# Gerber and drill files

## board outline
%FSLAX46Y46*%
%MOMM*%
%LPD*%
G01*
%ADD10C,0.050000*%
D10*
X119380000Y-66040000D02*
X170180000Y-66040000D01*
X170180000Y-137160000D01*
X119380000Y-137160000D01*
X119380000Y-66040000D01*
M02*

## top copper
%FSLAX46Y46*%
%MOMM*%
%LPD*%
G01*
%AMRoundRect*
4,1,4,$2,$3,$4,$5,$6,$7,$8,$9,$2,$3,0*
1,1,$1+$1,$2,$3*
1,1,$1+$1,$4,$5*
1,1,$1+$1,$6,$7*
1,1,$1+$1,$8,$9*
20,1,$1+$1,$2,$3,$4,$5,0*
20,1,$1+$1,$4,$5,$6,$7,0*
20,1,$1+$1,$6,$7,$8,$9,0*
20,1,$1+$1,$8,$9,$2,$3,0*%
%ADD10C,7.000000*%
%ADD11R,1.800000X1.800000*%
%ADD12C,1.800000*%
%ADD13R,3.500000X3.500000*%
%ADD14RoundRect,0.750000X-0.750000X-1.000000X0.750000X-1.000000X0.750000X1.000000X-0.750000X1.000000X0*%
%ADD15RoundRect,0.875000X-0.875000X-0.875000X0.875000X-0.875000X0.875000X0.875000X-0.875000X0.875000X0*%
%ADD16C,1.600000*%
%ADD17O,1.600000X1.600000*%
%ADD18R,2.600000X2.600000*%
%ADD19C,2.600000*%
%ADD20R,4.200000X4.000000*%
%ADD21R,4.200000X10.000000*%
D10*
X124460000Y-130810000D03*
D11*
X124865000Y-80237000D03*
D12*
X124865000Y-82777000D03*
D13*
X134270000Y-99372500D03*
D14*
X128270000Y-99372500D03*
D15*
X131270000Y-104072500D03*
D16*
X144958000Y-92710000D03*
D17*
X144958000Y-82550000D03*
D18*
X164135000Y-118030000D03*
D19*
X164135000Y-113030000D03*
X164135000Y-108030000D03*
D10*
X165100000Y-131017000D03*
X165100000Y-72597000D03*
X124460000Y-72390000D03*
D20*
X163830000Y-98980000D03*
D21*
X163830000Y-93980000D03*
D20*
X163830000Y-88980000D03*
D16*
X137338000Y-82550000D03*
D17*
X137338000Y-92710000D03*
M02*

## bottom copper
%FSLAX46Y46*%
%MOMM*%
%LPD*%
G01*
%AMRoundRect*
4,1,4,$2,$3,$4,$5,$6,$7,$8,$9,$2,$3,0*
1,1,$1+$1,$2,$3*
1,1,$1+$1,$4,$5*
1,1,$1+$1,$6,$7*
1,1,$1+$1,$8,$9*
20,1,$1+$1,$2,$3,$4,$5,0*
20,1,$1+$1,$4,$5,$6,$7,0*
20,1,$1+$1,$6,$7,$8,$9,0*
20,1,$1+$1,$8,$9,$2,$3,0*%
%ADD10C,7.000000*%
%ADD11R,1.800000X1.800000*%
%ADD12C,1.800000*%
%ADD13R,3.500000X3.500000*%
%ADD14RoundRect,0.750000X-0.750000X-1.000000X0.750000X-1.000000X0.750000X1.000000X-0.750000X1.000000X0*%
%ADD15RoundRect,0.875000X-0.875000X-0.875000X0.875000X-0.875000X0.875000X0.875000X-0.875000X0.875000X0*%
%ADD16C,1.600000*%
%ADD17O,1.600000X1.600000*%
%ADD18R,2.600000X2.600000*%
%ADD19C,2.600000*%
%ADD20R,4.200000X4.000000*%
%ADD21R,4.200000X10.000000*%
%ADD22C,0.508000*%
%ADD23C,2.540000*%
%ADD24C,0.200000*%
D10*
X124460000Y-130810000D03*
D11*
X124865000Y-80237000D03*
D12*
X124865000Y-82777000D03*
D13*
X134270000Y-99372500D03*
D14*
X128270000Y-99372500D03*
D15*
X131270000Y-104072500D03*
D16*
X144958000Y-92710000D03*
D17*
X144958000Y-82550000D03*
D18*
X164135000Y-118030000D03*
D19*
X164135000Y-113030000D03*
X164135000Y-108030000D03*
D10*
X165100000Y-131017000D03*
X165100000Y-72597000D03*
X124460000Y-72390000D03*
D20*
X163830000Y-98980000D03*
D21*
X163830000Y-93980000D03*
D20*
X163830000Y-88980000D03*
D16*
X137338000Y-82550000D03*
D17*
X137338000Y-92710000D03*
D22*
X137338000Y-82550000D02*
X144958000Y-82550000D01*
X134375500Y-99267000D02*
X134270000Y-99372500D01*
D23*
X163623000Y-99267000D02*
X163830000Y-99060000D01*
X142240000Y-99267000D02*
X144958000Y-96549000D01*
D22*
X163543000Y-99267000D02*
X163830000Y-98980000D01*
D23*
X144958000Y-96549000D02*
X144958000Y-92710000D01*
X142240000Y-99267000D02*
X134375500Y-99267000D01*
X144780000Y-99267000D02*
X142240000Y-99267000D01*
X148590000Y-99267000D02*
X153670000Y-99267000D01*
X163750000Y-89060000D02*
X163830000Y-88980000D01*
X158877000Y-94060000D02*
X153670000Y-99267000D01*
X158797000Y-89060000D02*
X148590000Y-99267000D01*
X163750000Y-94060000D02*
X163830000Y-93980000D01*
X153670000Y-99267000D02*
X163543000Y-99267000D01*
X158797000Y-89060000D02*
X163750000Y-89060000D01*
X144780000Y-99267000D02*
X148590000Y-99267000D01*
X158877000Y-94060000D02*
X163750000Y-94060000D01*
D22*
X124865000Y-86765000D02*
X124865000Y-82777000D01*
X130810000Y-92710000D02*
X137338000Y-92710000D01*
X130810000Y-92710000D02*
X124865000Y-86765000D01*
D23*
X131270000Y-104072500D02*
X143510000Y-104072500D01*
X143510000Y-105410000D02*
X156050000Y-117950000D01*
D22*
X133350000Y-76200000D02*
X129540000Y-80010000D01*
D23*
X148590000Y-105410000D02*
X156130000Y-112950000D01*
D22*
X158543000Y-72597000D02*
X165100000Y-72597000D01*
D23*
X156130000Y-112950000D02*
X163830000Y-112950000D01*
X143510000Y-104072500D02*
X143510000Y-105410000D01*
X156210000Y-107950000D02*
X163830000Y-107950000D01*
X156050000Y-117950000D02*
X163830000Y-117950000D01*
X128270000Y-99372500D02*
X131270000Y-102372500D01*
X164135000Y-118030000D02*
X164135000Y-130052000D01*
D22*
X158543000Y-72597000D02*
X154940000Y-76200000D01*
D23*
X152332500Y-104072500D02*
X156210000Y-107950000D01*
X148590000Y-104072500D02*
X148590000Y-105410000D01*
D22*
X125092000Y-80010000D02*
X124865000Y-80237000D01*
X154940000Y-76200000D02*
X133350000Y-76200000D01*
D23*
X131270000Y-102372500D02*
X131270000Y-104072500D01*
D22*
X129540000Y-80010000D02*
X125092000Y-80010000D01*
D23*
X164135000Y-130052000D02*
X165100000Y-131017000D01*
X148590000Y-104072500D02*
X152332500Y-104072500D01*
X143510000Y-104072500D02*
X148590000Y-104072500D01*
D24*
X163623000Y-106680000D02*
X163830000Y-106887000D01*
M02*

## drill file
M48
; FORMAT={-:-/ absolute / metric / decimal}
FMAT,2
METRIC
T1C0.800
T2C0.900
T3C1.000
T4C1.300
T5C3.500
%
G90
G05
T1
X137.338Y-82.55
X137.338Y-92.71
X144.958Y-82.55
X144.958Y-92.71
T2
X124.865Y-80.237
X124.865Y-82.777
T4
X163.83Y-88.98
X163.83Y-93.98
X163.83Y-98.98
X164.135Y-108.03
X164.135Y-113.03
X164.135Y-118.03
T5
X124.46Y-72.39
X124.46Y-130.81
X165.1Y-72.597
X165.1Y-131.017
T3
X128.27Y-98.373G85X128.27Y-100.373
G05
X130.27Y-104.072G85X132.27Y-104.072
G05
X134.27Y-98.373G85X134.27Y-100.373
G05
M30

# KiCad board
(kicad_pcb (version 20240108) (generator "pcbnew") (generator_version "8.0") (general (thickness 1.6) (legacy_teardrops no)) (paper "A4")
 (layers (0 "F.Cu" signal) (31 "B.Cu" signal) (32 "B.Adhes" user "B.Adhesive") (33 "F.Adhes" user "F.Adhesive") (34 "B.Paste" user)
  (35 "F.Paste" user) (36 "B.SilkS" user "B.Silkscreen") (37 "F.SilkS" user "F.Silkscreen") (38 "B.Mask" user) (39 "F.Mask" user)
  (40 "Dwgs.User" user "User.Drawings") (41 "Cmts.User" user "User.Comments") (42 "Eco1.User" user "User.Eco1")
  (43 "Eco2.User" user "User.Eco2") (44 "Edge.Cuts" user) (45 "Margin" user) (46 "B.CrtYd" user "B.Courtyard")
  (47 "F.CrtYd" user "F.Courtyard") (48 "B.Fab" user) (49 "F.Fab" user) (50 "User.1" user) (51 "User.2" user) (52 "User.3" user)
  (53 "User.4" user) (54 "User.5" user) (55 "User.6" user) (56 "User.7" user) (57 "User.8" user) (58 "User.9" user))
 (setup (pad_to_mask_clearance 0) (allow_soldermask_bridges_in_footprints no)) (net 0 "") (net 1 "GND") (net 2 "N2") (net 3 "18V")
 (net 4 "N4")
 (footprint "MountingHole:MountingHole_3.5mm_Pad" (layer "F.Cu") (at 124.46 130.81)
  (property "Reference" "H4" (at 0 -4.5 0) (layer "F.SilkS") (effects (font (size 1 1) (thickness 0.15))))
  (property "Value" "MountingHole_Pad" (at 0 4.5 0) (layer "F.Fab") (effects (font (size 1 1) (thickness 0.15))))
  (pad "1" thru_hole circle (at 0 0) (size 7 7) (drill 3.5) (layers "*.Cu" "*.Mask") (remove_unused_layers no) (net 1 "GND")))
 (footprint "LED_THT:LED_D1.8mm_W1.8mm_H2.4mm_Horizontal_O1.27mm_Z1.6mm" (layer "F.Cu") (at 124.865 80.237 -90)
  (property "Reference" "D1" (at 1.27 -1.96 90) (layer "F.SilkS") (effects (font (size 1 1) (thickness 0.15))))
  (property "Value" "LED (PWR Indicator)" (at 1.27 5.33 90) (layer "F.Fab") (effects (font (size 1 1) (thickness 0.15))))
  (pad "1" thru_hole rect (at 0 0 270) (size 1.8 1.8) (drill 0.9) (layers "*.Cu" "*.Mask") (remove_unused_layers no) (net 1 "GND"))
  (pad "2" thru_hole circle (at 2.54 0 270) (size 1.8 1.8) (drill 0.9) (layers "*.Cu" "*.Mask") (remove_unused_layers no) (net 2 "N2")))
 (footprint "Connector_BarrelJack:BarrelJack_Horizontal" (layer "F.Cu") (at 134.27 99.3725)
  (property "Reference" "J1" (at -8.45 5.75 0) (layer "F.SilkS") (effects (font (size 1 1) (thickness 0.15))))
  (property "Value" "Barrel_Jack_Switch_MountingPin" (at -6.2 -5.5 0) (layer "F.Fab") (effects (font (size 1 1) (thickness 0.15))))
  (pad "1" thru_hole rect (at 0 0) (size 3.5 3.5) (drill oval 1 3) (layers "*.Cu" "*.Mask") (remove_unused_layers no) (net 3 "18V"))
  (pad "2" thru_hole roundrect (at -6 0) (size 3 3.5) (drill oval 1 3) (layers "*.Cu" "*.Mask") (remove_unused_layers no)
   (roundrect_rratio 0.25) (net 1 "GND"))
  (pad "3" thru_hole roundrect (at -3 4.7) (size 3.5 3.5) (drill oval 3 1) (layers "*.Cu" "*.Mask") (remove_unused_layers no)
   (roundrect_rratio 0.25) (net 1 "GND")))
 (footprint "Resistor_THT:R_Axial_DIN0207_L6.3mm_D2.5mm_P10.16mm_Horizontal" (layer "F.Cu") (at 144.958 92.71 90)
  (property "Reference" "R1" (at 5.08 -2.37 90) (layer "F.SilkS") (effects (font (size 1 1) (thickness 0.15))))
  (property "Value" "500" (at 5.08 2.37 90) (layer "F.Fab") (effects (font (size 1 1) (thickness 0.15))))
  (pad "1" thru_hole circle (at 0 0 90) (size 1.6 1.6) (drill 0.8) (layers "*.Cu" "*.Mask") (remove_unused_layers no) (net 3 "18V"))
  (pad "2" thru_hole oval (at 10.16 0 90) (size 1.6 1.6) (drill 0.8) (layers "*.Cu" "*.Mask") (remove_unused_layers no) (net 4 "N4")))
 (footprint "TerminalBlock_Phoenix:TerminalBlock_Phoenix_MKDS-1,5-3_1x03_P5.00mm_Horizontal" (layer "F.Cu") (at 164.135 118.03 90)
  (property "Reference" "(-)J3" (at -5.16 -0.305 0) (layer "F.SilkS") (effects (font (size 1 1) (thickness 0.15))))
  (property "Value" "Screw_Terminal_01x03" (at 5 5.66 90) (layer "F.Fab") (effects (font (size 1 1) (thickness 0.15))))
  (pad "1" thru_hole rect (at 0 0 90) (size 2.6 2.6) (drill 1.3) (layers "*.Cu" "*.Mask") (remove_unused_layers no) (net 1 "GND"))
  (pad "2" thru_hole circle (at 5 0 90) (size 2.6 2.6) (drill 1.3) (layers "*.Cu" "*.Mask") (remove_unused_layers no) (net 1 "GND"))
  (pad "3" thru_hole circle (at 10 0 90) (size 2.6 2.6) (drill 1.3) (layers "*.Cu" "*.Mask") (remove_unused_layers no) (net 1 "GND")))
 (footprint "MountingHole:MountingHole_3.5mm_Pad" (layer "F.Cu") (at 165.1 131.017)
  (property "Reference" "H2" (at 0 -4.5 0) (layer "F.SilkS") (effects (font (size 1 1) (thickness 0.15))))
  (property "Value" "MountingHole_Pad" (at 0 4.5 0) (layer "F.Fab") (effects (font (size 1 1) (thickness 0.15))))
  (pad "1" thru_hole circle (at 0 0) (size 7 7) (drill 3.5) (layers "*.Cu" "*.Mask") (remove_unused_layers no) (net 1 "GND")))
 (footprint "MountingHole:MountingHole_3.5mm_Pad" (layer "F.Cu") (at 165.1 72.597)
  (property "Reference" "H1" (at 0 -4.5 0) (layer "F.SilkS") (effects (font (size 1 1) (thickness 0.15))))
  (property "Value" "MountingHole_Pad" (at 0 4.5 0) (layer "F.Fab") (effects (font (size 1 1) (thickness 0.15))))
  (pad "1" thru_hole circle (at 0 0) (size 7 7) (drill 3.5) (layers "*.Cu" "*.Mask") (remove_unused_layers no) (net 1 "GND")))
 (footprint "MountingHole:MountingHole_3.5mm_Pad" (layer "F.Cu") (at 124.46 72.39)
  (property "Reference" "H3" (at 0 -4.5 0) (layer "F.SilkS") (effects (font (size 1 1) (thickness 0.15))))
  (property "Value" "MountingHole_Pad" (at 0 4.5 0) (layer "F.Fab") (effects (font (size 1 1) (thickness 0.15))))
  (pad "1" thru_hole circle (at 0 0) (size 7 7) (drill 3.5) (layers "*.Cu" "*.Mask") (remove_unused_layers no) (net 1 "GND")))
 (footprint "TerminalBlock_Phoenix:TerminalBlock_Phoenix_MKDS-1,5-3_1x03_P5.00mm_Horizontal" (layer "F.Cu") (at 163.83 98.98 90)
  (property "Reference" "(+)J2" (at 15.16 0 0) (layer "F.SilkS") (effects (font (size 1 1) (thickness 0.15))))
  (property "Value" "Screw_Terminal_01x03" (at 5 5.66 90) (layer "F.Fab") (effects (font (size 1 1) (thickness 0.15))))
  (pad "1" thru_hole rect (at 0 0 90) (size 4 4.2) (drill 1.3) (layers "*.Cu" "*.Mask") (remove_unused_layers no) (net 3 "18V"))
  (pad "2" thru_hole rect (at 5 0 90) (size 10 4.2) (drill 1.3) (layers "*.Cu" "*.Mask") (remove_unused_layers no) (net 3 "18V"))
  (pad "3" thru_hole rect (at 10 0 90) (size 4 4.2) (drill 1.3) (layers "*.Cu" "*.Mask") (remove_unused_layers no) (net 3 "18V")))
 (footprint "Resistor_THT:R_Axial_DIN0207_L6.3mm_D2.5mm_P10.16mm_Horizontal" (layer "F.Cu") (at 137.338 82.55 -90)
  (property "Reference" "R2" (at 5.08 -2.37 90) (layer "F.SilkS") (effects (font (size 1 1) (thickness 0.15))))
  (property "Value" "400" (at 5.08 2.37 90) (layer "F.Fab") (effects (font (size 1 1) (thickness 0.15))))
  (pad "1" thru_hole circle (at 0 0 270) (size 1.6 1.6) (drill 0.8) (layers "*.Cu" "*.Mask") (remove_unused_layers no) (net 4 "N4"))
  (pad "2" thru_hole oval (at 10.16 0 270) (size 1.6 1.6) (drill 0.8) (layers "*.Cu" "*.Mask") (remove_unused_layers no) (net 2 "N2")))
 (gr_rect (start 119.38 66.04) (end 170.18 137.16) (stroke (width 0.05) (type default)) (fill none) (layer "Edge.Cuts"))
 (segment (start 137.338 82.55) (end 144.958 82.55) (width 0.508) (layer "B.Cu") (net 4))
 (segment (start 134.3755 99.267) (end 134.27 99.3725) (width 0.508) (layer "B.Cu") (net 3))
 (segment (start 163.623 99.267) (end 163.83 99.06) (width 2.54) (layer "B.Cu") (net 3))
 (segment (start 142.24 99.267) (end 144.958 96.549) (width 2.54) (layer "B.Cu") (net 3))
 (segment (start 163.543 99.267) (end 163.83 98.98) (width 0.508) (layer "B.Cu") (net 3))
 (segment (start 144.958 96.549) (end 144.958 92.71) (width 2.54) (layer "B.Cu") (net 3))
 (segment (start 142.24 99.267) (end 134.3755 99.267) (width 2.54) (layer "B.Cu") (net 3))
 (segment (start 144.78 99.267) (end 142.24 99.267) (width 2.54) (layer "B.Cu") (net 3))
 (segment (start 148.59 99.267) (end 153.67 99.267) (width 2.54) (layer "B.Cu") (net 3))
 (segment (start 163.75 89.06) (end 163.83 88.98) (width 2.54) (layer "B.Cu") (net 3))
 (segment (start 158.877 94.06) (end 153.67 99.267) (width 2.54) (layer "B.Cu") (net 3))
 (segment (start 158.797 89.06) (end 148.59 99.267) (width 2.54) (layer "B.Cu") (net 3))
 (segment (start 163.75 94.06) (end 163.83 93.98) (width 2.54) (layer "B.Cu") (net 3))
 (segment (start 153.67 99.267) (end 163.543 99.267) (width 2.54) (layer "B.Cu") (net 3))
 (segment (start 158.797 89.06) (end 163.75 89.06) (width 2.54) (layer "B.Cu") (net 3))
 (segment (start 144.78 99.267) (end 148.59 99.267) (width 2.54) (layer "B.Cu") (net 3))
 (segment (start 158.877 94.06) (end 163.75 94.06) (width 2.54) (layer "B.Cu") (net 3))
 (segment (start 124.865 86.765) (end 124.865 82.777) (width 0.508) (layer "B.Cu") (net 2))
 (segment (start 130.81 92.71) (end 137.338 92.71) (width 0.508) (layer "B.Cu") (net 2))
 (segment (start 130.81 92.71) (end 124.865 86.765) (width 0.508) (layer "B.Cu") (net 2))
 (segment (start 131.27 104.0725) (end 143.51 104.0725) (width 2.54) (layer "B.Cu") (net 1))
 (segment (start 143.51 105.41) (end 156.05 117.95) (width 2.54) (layer "B.Cu") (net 1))
 (segment (start 133.35 76.2) (end 129.54 80.01) (width 0.508) (layer "B.Cu") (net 1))
 (segment (start 148.59 105.41) (end 156.13 112.95) (width 2.54) (layer "B.Cu") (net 1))
 (segment (start 158.543 72.597) (end 165.1 72.597) (width 0.508) (layer "B.Cu") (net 1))
 (segment (start 156.13 112.95) (end 163.83 112.95) (width 2.54) (layer "B.Cu") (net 1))
 (segment (start 143.51 104.0725) (end 143.51 105.41) (width 2.54) (layer "B.Cu") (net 1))
 (segment (start 156.21 107.95) (end 163.83 107.95) (width 2.54) (layer "B.Cu") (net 1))
 (segment (start 156.05 117.95) (end 163.83 117.95) (width 2.54) (layer "B.Cu") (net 1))
 (segment (start 128.27 99.3725) (end 131.27 102.3725) (width 2.54) (layer "B.Cu") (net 1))
 (segment (start 164.135 118.03) (end 164.135 130.052) (width 2.54) (layer "B.Cu") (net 1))
 (segment (start 158.543 72.597) (end 154.94 76.2) (width 0.508) (layer "B.Cu") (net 1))
 (segment (start 152.3325 104.0725) (end 156.21 107.95) (width 2.54) (layer "B.Cu") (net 1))
 (segment (start 148.59 104.0725) (end 148.59 105.41) (width 2.54) (layer "B.Cu") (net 1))
 (segment (start 125.092 80.01) (end 124.865 80.237) (width 0.508) (layer "B.Cu") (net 1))
 (segment (start 154.94 76.2) (end 133.35 76.2) (width 0.508) (layer "B.Cu") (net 1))
 (segment (start 131.27 102.3725) (end 131.27 104.0725) (width 2.54) (layer "B.Cu") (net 1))
 (segment (start 129.54 80.01) (end 125.092 80.01) (width 0.508) (layer "B.Cu") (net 1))
 (segment (start 164.135 130.052) (end 165.1 131.017) (width 2.54) (layer "B.Cu") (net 1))
 (segment (start 148.59 104.0725) (end 152.3325 104.0725) (width 2.54) (layer "B.Cu") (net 1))
 (segment (start 143.51 104.0725) (end 148.59 104.0725) (width 2.54) (layer "B.Cu") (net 1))
 (segment (start 163.623 106.68) (end 163.83 106.887) (width 0.2) (layer "B.Cu") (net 1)))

